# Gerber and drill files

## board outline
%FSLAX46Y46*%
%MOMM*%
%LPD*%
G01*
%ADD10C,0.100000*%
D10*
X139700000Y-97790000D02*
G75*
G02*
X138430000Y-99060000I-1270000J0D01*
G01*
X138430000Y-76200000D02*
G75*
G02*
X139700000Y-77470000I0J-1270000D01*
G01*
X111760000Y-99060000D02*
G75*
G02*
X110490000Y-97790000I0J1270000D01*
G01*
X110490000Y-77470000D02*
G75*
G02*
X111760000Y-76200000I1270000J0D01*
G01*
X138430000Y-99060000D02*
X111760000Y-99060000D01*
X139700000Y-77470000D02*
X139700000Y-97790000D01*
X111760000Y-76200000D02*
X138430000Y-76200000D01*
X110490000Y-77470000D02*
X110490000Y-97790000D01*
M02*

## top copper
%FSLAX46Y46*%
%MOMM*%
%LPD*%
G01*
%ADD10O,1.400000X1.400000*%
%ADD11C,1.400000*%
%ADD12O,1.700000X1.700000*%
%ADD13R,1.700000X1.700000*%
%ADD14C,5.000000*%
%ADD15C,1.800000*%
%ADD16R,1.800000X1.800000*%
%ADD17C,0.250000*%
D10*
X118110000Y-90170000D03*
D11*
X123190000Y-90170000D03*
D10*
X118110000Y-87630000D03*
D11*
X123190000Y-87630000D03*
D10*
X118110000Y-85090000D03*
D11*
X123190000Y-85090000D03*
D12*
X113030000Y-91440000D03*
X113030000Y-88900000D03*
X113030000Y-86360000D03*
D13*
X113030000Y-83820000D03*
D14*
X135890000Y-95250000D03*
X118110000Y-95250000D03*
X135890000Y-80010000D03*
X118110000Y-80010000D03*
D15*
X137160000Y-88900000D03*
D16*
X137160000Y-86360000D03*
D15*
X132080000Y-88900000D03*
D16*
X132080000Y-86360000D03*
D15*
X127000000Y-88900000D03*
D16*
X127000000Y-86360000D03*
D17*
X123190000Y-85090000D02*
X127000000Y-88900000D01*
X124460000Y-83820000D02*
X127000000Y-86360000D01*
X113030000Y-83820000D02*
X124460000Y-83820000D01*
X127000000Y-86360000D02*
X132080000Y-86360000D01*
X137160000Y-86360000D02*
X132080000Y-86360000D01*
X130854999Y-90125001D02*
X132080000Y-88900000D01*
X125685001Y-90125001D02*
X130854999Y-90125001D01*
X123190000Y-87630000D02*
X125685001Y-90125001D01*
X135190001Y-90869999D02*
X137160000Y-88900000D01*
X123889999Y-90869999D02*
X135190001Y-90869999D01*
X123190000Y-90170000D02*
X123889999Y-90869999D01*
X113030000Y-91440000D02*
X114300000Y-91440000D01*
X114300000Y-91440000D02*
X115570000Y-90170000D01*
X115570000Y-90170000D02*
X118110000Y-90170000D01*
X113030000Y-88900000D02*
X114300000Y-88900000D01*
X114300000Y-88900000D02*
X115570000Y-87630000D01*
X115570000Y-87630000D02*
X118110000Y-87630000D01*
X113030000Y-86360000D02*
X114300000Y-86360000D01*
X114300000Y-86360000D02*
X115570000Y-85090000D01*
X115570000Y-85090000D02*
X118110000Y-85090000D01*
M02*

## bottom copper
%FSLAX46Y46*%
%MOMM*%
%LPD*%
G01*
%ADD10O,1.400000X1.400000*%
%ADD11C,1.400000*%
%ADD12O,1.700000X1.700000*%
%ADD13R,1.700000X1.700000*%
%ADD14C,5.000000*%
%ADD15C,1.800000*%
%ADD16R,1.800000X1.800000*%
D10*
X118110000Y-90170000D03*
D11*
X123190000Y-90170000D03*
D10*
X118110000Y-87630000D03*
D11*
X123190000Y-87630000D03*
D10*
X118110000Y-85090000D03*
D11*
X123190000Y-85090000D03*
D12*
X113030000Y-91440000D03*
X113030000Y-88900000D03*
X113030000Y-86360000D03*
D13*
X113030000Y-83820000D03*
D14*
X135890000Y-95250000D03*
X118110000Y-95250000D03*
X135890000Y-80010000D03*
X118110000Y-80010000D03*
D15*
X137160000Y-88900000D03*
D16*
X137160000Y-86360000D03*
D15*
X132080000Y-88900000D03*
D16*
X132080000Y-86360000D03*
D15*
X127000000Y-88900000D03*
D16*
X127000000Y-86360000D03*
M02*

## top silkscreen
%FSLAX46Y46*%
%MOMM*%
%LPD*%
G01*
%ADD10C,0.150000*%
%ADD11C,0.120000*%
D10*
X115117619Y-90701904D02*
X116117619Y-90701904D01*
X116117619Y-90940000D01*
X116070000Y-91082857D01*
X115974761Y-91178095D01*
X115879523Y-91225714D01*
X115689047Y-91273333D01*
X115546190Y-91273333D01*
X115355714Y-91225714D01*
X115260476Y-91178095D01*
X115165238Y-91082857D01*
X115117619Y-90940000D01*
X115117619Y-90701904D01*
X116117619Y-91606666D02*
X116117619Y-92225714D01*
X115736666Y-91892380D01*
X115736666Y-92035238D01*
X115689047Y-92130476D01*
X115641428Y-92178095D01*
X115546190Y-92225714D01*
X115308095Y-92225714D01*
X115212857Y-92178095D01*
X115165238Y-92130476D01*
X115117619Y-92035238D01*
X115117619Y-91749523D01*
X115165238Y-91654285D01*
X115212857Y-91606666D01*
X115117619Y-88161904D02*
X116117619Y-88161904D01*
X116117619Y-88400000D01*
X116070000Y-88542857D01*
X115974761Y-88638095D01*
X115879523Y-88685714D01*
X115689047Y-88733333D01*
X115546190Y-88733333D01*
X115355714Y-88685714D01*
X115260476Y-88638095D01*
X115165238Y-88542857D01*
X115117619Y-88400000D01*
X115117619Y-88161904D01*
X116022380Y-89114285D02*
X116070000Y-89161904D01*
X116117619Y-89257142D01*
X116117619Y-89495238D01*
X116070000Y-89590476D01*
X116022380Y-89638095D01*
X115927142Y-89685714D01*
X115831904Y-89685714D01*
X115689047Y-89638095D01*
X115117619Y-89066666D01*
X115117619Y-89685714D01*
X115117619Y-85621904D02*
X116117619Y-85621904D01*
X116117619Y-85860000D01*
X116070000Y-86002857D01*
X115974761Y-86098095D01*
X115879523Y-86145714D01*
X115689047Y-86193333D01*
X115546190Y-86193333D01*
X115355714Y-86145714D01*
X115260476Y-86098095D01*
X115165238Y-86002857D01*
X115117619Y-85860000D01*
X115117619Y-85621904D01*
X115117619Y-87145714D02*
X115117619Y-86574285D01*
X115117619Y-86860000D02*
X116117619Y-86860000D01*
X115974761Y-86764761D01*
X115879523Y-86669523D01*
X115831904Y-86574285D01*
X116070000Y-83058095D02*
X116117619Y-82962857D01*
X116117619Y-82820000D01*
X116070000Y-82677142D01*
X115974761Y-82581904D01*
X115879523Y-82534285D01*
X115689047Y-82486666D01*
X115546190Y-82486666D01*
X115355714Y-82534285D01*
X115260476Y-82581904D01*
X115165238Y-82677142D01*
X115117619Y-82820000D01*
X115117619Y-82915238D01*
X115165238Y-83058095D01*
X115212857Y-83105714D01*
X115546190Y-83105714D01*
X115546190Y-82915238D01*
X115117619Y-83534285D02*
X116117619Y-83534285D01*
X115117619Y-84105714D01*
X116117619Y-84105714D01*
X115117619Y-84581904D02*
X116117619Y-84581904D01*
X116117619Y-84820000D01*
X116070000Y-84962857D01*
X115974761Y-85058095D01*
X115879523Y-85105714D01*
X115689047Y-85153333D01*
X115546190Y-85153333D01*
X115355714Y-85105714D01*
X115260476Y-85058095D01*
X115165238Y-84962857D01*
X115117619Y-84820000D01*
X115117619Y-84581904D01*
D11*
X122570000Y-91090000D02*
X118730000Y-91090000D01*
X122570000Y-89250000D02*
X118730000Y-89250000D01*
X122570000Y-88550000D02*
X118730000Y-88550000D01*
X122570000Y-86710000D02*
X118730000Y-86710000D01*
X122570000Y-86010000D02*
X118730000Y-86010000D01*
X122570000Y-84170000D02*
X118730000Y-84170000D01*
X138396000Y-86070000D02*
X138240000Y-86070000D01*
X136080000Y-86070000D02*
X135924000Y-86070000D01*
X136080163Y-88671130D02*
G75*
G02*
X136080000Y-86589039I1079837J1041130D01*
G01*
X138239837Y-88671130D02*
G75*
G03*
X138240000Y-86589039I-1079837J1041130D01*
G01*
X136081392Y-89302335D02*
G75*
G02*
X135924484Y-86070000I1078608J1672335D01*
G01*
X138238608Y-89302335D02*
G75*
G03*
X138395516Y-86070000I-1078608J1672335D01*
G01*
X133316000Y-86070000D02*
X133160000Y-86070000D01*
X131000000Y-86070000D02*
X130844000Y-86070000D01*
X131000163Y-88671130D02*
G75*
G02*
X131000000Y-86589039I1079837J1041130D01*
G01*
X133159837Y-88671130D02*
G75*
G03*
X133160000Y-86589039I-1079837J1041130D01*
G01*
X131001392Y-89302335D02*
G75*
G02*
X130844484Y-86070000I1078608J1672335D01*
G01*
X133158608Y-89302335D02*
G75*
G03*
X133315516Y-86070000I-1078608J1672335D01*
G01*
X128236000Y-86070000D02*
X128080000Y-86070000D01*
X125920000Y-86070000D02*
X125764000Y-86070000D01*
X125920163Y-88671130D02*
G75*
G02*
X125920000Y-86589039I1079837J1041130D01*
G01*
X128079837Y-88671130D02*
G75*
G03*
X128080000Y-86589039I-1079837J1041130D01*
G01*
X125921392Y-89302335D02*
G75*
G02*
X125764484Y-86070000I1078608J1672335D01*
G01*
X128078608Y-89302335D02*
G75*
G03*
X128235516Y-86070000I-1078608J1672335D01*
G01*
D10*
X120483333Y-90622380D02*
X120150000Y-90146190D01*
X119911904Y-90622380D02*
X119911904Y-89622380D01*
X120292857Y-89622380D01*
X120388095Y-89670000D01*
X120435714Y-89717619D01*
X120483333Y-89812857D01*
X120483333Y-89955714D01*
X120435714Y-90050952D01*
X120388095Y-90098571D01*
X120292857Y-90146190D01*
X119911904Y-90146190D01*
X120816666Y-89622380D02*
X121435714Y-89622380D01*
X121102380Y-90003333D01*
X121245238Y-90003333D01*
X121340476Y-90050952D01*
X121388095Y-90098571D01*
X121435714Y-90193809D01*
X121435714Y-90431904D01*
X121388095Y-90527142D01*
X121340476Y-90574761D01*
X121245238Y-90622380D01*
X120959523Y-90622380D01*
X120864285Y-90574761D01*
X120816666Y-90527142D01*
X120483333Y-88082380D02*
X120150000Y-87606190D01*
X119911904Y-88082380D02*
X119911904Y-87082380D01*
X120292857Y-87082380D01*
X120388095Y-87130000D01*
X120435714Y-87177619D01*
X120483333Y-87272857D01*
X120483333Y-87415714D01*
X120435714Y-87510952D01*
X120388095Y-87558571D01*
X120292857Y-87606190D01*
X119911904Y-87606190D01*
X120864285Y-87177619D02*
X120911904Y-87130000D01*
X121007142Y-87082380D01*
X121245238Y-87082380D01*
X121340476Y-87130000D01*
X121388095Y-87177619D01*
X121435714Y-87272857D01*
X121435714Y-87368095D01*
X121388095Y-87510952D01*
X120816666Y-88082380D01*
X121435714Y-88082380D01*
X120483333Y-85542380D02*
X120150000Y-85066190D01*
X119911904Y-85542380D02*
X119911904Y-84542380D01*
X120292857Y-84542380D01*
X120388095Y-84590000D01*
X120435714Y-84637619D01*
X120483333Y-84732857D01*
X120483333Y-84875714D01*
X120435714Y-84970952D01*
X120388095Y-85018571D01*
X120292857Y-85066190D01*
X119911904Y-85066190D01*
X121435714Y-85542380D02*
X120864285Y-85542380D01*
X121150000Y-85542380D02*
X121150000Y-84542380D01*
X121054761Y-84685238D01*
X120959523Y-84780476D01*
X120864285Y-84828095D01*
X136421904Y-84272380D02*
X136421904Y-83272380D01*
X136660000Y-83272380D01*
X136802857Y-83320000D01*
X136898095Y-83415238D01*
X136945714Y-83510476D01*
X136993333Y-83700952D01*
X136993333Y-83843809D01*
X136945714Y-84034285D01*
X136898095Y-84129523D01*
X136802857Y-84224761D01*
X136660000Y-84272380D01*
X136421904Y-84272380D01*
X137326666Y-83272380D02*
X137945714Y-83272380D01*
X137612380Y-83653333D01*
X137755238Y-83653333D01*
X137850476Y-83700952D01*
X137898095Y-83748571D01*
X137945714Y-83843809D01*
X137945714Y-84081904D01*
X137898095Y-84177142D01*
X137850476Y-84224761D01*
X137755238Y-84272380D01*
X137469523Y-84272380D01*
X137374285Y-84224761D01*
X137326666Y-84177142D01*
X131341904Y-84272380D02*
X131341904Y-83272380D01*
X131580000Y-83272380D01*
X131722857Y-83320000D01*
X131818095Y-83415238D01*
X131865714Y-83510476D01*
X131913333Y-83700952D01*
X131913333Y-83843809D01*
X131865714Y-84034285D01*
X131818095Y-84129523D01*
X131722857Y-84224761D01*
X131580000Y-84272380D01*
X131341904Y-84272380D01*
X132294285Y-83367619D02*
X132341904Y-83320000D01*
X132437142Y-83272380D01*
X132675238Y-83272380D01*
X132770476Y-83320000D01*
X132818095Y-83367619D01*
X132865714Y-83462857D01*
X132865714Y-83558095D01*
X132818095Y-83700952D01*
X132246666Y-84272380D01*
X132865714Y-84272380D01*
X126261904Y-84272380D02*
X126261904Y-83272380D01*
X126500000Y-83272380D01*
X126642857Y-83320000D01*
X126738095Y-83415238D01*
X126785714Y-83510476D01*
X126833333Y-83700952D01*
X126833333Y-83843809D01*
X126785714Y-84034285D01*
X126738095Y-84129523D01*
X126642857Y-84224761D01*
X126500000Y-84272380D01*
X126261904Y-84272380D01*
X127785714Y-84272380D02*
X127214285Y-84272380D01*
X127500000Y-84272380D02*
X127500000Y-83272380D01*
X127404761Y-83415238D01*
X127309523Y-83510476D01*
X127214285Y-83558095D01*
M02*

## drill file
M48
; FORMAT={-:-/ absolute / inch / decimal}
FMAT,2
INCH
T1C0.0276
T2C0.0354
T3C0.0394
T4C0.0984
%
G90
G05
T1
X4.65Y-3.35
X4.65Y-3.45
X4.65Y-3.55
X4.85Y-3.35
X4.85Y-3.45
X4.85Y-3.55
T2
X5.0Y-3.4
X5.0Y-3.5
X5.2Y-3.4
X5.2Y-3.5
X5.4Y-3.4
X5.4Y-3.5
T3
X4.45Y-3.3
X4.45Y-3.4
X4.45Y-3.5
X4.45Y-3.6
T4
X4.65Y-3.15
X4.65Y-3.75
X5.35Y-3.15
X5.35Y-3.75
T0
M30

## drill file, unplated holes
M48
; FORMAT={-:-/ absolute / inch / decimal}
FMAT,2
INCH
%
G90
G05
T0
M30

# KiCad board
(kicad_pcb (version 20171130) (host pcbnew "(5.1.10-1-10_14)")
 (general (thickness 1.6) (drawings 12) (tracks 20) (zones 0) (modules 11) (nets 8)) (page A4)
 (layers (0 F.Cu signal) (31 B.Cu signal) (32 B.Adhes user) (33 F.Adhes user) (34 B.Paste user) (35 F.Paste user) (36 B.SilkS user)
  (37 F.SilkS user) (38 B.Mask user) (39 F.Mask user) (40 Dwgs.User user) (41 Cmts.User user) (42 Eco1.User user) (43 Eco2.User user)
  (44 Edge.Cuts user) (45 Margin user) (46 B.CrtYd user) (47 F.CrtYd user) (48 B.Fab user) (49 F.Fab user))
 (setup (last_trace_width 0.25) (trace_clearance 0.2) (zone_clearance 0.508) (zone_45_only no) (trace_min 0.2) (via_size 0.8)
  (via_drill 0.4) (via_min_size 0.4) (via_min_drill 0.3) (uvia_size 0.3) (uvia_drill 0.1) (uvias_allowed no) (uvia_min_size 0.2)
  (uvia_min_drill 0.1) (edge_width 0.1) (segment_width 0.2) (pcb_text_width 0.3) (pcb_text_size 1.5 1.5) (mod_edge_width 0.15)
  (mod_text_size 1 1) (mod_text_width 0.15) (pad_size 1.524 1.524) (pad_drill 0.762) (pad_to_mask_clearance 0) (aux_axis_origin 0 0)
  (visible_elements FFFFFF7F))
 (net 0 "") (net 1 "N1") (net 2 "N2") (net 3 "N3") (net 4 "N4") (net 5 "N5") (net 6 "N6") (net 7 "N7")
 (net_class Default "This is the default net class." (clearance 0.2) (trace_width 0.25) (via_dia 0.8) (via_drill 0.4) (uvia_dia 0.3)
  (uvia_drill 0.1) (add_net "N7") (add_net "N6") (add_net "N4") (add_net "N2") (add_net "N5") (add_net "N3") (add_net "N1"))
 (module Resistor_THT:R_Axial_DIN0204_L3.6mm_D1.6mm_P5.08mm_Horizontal (layer F.Cu) (at 123.19 90.17 180)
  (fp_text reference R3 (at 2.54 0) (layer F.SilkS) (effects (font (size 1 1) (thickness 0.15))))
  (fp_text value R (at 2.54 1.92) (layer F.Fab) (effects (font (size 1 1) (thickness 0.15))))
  (fp_line (start 0.62 -0.92) (end 4.46 -0.92) (layer F.SilkS) (width 0.12))
  (fp_line (start 0.62 0.92) (end 4.46 0.92) (layer F.SilkS) (width 0.12))
  (pad 2 thru_hole oval (at 5.08 0 180) (size 1.4 1.4) (drill 0.7) (layers *.Cu *.Mask) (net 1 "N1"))
  (pad 1 thru_hole circle (at 0 0 180) (size 1.4 1.4) (drill 0.7) (layers *.Cu *.Mask) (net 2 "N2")))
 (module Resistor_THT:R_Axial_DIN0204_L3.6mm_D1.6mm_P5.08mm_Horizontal (layer F.Cu) (at 123.19 87.63 180)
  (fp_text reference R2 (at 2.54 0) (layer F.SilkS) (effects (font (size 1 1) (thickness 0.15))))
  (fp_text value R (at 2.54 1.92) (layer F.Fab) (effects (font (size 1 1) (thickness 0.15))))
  (fp_line (start 0.62 -0.92) (end 4.46 -0.92) (layer F.SilkS) (width 0.12))
  (fp_line (start 0.62 0.92) (end 4.46 0.92) (layer F.SilkS) (width 0.12))
  (pad 2 thru_hole oval (at 5.08 0 180) (size 1.4 1.4) (drill 0.7) (layers *.Cu *.Mask) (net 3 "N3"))
  (pad 1 thru_hole circle (at 0 0 180) (size 1.4 1.4) (drill 0.7) (layers *.Cu *.Mask) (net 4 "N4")))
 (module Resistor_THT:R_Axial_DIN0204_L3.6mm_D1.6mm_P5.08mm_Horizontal (layer F.Cu) (at 123.19 85.09 180)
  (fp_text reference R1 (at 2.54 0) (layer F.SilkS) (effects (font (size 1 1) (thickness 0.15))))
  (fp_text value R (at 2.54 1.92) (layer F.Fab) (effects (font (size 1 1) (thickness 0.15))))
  (fp_line (start 0.62 -0.92) (end 4.46 -0.92) (layer F.SilkS) (width 0.12))
  (fp_line (start 0.62 0.92) (end 4.46 0.92) (layer F.SilkS) (width 0.12))
  (pad 2 thru_hole oval (at 5.08 0 180) (size 1.4 1.4) (drill 0.7) (layers *.Cu *.Mask) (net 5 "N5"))
  (pad 1 thru_hole circle (at 0 0 180) (size 1.4 1.4) (drill 0.7) (layers *.Cu *.Mask) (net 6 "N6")))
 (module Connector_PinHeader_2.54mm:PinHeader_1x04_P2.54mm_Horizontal (layer B.Cu) (at 113.03 83.82 180)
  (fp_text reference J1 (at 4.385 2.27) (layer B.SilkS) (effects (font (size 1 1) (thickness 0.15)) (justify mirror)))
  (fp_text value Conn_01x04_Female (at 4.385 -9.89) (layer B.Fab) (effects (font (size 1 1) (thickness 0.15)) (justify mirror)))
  (pad 4 thru_hole oval (at 0 -7.62 180) (size 1.7 1.7) (drill 1) (layers *.Cu *.Mask) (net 1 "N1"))
  (pad 3 thru_hole oval (at 0 -5.08 180) (size 1.7 1.7) (drill 1) (layers *.Cu *.Mask) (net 3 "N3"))
  (pad 2 thru_hole oval (at 0 -2.54 180) (size 1.7 1.7) (drill 1) (layers *.Cu *.Mask) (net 5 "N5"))
  (pad 1 thru_hole rect (at 0 0 180) (size 1.7 1.7) (drill 1) (layers *.Cu *.Mask) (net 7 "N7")))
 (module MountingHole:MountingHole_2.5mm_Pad (layer F.Cu) (at 135.89 95.25)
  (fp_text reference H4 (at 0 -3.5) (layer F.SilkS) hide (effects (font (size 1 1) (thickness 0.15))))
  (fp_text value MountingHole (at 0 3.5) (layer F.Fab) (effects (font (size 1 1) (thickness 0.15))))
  (pad 1 thru_hole circle (at 0 0) (size 5 5) (drill 2.5) (layers *.Cu *.Mask)))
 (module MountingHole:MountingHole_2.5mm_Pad (layer F.Cu) (at 118.11 95.25)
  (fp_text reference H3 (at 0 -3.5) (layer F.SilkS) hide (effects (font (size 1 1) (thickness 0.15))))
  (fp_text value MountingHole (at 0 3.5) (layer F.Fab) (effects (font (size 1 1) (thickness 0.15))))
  (pad 1 thru_hole circle (at 0 0) (size 5 5) (drill 2.5) (layers *.Cu *.Mask)))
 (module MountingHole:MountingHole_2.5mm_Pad (layer F.Cu) (at 135.89 80.01)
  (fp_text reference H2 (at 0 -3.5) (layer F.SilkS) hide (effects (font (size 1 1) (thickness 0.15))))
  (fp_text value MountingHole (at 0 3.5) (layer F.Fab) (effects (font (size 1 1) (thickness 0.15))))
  (pad 1 thru_hole circle (at 0 0) (size 5 5) (drill 2.5) (layers *.Cu *.Mask)))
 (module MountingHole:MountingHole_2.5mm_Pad (layer F.Cu) (at 118.11 80.01)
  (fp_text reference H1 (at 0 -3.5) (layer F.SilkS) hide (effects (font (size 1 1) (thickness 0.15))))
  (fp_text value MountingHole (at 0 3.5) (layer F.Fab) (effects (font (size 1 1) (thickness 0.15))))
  (pad 1 thru_hole circle (at 0 0) (size 5 5) (drill 2.5) (layers *.Cu *.Mask)))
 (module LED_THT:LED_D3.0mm (layer F.Cu) (at 137.16 86.36 270)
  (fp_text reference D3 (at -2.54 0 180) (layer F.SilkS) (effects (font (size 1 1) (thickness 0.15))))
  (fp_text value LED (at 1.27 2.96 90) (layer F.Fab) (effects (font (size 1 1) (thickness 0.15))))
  (fp_line (start -0.29 -1.236) (end -0.29 -1.08) (layer F.SilkS) (width 0.12))
  (fp_line (start -0.29 1.08) (end -0.29 1.236) (layer F.SilkS) (width 0.12))
  (fp_arc (start 1.27 0) (end 0.229039 1.08) (angle -87.9) (layer F.SilkS) (width 0.12))
  (fp_arc (start 1.27 0) (end 0.229039 -1.08) (angle 87.9) (layer F.SilkS) (width 0.12))
  (fp_arc (start 1.27 0) (end -0.29 1.235516) (angle -108.8) (layer F.SilkS) (width 0.12))
  (fp_arc (start 1.27 0) (end -0.29 -1.235516) (angle 108.8) (layer F.SilkS) (width 0.12))
  (pad 2 thru_hole circle (at 2.54 0 270) (size 1.8 1.8) (drill 0.9) (layers *.Cu *.Mask) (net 2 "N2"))
  (pad 1 thru_hole rect (at 0 0 270) (size 1.8 1.8) (drill 0.9) (layers *.Cu *.Mask) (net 7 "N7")))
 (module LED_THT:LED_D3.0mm (layer F.Cu) (at 132.08 86.36 270)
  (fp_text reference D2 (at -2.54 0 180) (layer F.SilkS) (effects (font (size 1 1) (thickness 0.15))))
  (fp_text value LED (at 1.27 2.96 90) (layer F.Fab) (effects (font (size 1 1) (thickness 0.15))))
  (fp_line (start -0.29 -1.236) (end -0.29 -1.08) (layer F.SilkS) (width 0.12))
  (fp_line (start -0.29 1.08) (end -0.29 1.236) (layer F.SilkS) (width 0.12))
  (fp_arc (start 1.27 0) (end 0.229039 1.08) (angle -87.9) (layer F.SilkS) (width 0.12))
  (fp_arc (start 1.27 0) (end 0.229039 -1.08) (angle 87.9) (layer F.SilkS) (width 0.12))
  (fp_arc (start 1.27 0) (end -0.29 1.235516) (angle -108.8) (layer F.SilkS) (width 0.12))
  (fp_arc (start 1.27 0) (end -0.29 -1.235516) (angle 108.8) (layer F.SilkS) (width 0.12))
  (pad 2 thru_hole circle (at 2.54 0 270) (size 1.8 1.8) (drill 0.9) (layers *.Cu *.Mask) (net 4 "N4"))
  (pad 1 thru_hole rect (at 0 0 270) (size 1.8 1.8) (drill 0.9) (layers *.Cu *.Mask) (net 7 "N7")))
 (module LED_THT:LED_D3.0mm (layer F.Cu) (at 127 86.36 270)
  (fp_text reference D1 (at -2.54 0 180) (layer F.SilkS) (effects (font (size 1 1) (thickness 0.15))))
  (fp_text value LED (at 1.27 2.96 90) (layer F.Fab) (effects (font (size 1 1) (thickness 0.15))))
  (fp_line (start -0.29 -1.236) (end -0.29 -1.08) (layer F.SilkS) (width 0.12))
  (fp_line (start -0.29 1.08) (end -0.29 1.236) (layer F.SilkS) (width 0.12))
  (fp_arc (start 1.27 0) (end 0.229039 1.08) (angle -87.9) (layer F.SilkS) (width 0.12))
  (fp_arc (start 1.27 0) (end 0.229039 -1.08) (angle 87.9) (layer F.SilkS) (width 0.12))
  (fp_arc (start 1.27 0) (end -0.29 1.235516) (angle -108.8) (layer F.SilkS) (width 0.12))
  (fp_arc (start 1.27 0) (end -0.29 -1.235516) (angle 108.8) (layer F.SilkS) (width 0.12))
  (pad 2 thru_hole circle (at 2.54 0 270) (size 1.8 1.8) (drill 0.9) (layers *.Cu *.Mask) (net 6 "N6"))
  (pad 1 thru_hole rect (at 0 0 270) (size 1.8 1.8) (drill 0.9) (layers *.Cu *.Mask) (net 7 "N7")))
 (gr_arc (start 138.43 97.79) (end 138.43 99.06) (angle -90) (layer Edge.Cuts) (width 0.1))
 (gr_arc (start 138.43 77.47) (end 139.7 77.47) (angle -90) (layer Edge.Cuts) (width 0.1))
 (gr_arc (start 111.76 97.79) (end 110.49 97.79) (angle -90) (layer Edge.Cuts) (width 0.1))
 (gr_arc (start 111.76 77.47) (end 111.76 76.2) (angle -90) (layer Edge.Cuts) (width 0.1))
 (gr_line (start 138.43 99.06) (end 111.76 99.06) (layer Edge.Cuts) (width 0.1))
 (gr_line (start 139.7 77.47) (end 139.7 97.79) (layer Edge.Cuts) (width 0.1))
 (gr_line (start 111.76 76.2) (end 138.43 76.2) (layer Edge.Cuts) (width 0.1))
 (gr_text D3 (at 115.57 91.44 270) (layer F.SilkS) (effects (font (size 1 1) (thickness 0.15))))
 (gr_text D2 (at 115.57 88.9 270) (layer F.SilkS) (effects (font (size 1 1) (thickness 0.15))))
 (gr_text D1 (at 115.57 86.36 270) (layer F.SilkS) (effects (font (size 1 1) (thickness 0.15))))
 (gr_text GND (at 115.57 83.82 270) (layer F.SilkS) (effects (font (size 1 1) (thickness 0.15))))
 (gr_line (start 110.49 77.47) (end 110.49 97.79) (layer Edge.Cuts) (width 0.1))
 (segment (start 123.19 85.09) (end 127 88.9) (width 0.25) (layer F.Cu) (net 6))
 (segment (start 124.46 83.82) (end 127 86.36) (width 0.25) (layer F.Cu) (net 7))
 (segment (start 113.03 83.82) (end 124.46 83.82) (width 0.25) (layer F.Cu) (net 7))
 (segment (start 127 86.36) (end 132.08 86.36) (width 0.25) (layer F.Cu) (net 7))
 (segment (start 137.16 86.36) (end 132.08 86.36) (width 0.25) (layer F.Cu) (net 7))
 (segment (start 130.854999 90.125001) (end 132.08 88.9) (width 0.25) (layer F.Cu) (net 4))
 (segment (start 125.685001 90.125001) (end 130.854999 90.125001) (width 0.25) (layer F.Cu) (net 4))
 (segment (start 123.19 87.63) (end 125.685001 90.125001) (width 0.25) (layer F.Cu) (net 4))
 (segment (start 135.190001 90.869999) (end 137.16 88.9) (width 0.25) (layer F.Cu) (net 2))
 (segment (start 123.889999 90.869999) (end 135.190001 90.869999) (width 0.25) (layer F.Cu) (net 2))
 (segment (start 123.19 90.17) (end 123.889999 90.869999) (width 0.25) (layer F.Cu) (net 2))
 (segment (start 113.03 91.44) (end 114.3 91.44) (width 0.25) (layer F.Cu) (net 1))
 (segment (start 114.3 91.44) (end 115.57 90.17) (width 0.25) (layer F.Cu) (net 1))
 (segment (start 115.57 90.17) (end 118.11 90.17) (width 0.25) (layer F.Cu) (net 1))
 (segment (start 113.03 88.9) (end 114.3 88.9) (width 0.25) (layer F.Cu) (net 3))
 (segment (start 114.3 88.9) (end 115.57 87.63) (width 0.25) (layer F.Cu) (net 3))
 (segment (start 115.57 87.63) (end 118.11 87.63) (width 0.25) (layer F.Cu) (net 3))
 (segment (start 113.03 86.36) (end 114.3 86.36) (width 0.25) (layer F.Cu) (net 5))
 (segment (start 114.3 86.36) (end 115.57 85.09) (width 0.25) (layer F.Cu) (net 5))
 (segment (start 115.57 85.09) (end 118.11 85.09) (width 0.25) (layer F.Cu) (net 5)))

